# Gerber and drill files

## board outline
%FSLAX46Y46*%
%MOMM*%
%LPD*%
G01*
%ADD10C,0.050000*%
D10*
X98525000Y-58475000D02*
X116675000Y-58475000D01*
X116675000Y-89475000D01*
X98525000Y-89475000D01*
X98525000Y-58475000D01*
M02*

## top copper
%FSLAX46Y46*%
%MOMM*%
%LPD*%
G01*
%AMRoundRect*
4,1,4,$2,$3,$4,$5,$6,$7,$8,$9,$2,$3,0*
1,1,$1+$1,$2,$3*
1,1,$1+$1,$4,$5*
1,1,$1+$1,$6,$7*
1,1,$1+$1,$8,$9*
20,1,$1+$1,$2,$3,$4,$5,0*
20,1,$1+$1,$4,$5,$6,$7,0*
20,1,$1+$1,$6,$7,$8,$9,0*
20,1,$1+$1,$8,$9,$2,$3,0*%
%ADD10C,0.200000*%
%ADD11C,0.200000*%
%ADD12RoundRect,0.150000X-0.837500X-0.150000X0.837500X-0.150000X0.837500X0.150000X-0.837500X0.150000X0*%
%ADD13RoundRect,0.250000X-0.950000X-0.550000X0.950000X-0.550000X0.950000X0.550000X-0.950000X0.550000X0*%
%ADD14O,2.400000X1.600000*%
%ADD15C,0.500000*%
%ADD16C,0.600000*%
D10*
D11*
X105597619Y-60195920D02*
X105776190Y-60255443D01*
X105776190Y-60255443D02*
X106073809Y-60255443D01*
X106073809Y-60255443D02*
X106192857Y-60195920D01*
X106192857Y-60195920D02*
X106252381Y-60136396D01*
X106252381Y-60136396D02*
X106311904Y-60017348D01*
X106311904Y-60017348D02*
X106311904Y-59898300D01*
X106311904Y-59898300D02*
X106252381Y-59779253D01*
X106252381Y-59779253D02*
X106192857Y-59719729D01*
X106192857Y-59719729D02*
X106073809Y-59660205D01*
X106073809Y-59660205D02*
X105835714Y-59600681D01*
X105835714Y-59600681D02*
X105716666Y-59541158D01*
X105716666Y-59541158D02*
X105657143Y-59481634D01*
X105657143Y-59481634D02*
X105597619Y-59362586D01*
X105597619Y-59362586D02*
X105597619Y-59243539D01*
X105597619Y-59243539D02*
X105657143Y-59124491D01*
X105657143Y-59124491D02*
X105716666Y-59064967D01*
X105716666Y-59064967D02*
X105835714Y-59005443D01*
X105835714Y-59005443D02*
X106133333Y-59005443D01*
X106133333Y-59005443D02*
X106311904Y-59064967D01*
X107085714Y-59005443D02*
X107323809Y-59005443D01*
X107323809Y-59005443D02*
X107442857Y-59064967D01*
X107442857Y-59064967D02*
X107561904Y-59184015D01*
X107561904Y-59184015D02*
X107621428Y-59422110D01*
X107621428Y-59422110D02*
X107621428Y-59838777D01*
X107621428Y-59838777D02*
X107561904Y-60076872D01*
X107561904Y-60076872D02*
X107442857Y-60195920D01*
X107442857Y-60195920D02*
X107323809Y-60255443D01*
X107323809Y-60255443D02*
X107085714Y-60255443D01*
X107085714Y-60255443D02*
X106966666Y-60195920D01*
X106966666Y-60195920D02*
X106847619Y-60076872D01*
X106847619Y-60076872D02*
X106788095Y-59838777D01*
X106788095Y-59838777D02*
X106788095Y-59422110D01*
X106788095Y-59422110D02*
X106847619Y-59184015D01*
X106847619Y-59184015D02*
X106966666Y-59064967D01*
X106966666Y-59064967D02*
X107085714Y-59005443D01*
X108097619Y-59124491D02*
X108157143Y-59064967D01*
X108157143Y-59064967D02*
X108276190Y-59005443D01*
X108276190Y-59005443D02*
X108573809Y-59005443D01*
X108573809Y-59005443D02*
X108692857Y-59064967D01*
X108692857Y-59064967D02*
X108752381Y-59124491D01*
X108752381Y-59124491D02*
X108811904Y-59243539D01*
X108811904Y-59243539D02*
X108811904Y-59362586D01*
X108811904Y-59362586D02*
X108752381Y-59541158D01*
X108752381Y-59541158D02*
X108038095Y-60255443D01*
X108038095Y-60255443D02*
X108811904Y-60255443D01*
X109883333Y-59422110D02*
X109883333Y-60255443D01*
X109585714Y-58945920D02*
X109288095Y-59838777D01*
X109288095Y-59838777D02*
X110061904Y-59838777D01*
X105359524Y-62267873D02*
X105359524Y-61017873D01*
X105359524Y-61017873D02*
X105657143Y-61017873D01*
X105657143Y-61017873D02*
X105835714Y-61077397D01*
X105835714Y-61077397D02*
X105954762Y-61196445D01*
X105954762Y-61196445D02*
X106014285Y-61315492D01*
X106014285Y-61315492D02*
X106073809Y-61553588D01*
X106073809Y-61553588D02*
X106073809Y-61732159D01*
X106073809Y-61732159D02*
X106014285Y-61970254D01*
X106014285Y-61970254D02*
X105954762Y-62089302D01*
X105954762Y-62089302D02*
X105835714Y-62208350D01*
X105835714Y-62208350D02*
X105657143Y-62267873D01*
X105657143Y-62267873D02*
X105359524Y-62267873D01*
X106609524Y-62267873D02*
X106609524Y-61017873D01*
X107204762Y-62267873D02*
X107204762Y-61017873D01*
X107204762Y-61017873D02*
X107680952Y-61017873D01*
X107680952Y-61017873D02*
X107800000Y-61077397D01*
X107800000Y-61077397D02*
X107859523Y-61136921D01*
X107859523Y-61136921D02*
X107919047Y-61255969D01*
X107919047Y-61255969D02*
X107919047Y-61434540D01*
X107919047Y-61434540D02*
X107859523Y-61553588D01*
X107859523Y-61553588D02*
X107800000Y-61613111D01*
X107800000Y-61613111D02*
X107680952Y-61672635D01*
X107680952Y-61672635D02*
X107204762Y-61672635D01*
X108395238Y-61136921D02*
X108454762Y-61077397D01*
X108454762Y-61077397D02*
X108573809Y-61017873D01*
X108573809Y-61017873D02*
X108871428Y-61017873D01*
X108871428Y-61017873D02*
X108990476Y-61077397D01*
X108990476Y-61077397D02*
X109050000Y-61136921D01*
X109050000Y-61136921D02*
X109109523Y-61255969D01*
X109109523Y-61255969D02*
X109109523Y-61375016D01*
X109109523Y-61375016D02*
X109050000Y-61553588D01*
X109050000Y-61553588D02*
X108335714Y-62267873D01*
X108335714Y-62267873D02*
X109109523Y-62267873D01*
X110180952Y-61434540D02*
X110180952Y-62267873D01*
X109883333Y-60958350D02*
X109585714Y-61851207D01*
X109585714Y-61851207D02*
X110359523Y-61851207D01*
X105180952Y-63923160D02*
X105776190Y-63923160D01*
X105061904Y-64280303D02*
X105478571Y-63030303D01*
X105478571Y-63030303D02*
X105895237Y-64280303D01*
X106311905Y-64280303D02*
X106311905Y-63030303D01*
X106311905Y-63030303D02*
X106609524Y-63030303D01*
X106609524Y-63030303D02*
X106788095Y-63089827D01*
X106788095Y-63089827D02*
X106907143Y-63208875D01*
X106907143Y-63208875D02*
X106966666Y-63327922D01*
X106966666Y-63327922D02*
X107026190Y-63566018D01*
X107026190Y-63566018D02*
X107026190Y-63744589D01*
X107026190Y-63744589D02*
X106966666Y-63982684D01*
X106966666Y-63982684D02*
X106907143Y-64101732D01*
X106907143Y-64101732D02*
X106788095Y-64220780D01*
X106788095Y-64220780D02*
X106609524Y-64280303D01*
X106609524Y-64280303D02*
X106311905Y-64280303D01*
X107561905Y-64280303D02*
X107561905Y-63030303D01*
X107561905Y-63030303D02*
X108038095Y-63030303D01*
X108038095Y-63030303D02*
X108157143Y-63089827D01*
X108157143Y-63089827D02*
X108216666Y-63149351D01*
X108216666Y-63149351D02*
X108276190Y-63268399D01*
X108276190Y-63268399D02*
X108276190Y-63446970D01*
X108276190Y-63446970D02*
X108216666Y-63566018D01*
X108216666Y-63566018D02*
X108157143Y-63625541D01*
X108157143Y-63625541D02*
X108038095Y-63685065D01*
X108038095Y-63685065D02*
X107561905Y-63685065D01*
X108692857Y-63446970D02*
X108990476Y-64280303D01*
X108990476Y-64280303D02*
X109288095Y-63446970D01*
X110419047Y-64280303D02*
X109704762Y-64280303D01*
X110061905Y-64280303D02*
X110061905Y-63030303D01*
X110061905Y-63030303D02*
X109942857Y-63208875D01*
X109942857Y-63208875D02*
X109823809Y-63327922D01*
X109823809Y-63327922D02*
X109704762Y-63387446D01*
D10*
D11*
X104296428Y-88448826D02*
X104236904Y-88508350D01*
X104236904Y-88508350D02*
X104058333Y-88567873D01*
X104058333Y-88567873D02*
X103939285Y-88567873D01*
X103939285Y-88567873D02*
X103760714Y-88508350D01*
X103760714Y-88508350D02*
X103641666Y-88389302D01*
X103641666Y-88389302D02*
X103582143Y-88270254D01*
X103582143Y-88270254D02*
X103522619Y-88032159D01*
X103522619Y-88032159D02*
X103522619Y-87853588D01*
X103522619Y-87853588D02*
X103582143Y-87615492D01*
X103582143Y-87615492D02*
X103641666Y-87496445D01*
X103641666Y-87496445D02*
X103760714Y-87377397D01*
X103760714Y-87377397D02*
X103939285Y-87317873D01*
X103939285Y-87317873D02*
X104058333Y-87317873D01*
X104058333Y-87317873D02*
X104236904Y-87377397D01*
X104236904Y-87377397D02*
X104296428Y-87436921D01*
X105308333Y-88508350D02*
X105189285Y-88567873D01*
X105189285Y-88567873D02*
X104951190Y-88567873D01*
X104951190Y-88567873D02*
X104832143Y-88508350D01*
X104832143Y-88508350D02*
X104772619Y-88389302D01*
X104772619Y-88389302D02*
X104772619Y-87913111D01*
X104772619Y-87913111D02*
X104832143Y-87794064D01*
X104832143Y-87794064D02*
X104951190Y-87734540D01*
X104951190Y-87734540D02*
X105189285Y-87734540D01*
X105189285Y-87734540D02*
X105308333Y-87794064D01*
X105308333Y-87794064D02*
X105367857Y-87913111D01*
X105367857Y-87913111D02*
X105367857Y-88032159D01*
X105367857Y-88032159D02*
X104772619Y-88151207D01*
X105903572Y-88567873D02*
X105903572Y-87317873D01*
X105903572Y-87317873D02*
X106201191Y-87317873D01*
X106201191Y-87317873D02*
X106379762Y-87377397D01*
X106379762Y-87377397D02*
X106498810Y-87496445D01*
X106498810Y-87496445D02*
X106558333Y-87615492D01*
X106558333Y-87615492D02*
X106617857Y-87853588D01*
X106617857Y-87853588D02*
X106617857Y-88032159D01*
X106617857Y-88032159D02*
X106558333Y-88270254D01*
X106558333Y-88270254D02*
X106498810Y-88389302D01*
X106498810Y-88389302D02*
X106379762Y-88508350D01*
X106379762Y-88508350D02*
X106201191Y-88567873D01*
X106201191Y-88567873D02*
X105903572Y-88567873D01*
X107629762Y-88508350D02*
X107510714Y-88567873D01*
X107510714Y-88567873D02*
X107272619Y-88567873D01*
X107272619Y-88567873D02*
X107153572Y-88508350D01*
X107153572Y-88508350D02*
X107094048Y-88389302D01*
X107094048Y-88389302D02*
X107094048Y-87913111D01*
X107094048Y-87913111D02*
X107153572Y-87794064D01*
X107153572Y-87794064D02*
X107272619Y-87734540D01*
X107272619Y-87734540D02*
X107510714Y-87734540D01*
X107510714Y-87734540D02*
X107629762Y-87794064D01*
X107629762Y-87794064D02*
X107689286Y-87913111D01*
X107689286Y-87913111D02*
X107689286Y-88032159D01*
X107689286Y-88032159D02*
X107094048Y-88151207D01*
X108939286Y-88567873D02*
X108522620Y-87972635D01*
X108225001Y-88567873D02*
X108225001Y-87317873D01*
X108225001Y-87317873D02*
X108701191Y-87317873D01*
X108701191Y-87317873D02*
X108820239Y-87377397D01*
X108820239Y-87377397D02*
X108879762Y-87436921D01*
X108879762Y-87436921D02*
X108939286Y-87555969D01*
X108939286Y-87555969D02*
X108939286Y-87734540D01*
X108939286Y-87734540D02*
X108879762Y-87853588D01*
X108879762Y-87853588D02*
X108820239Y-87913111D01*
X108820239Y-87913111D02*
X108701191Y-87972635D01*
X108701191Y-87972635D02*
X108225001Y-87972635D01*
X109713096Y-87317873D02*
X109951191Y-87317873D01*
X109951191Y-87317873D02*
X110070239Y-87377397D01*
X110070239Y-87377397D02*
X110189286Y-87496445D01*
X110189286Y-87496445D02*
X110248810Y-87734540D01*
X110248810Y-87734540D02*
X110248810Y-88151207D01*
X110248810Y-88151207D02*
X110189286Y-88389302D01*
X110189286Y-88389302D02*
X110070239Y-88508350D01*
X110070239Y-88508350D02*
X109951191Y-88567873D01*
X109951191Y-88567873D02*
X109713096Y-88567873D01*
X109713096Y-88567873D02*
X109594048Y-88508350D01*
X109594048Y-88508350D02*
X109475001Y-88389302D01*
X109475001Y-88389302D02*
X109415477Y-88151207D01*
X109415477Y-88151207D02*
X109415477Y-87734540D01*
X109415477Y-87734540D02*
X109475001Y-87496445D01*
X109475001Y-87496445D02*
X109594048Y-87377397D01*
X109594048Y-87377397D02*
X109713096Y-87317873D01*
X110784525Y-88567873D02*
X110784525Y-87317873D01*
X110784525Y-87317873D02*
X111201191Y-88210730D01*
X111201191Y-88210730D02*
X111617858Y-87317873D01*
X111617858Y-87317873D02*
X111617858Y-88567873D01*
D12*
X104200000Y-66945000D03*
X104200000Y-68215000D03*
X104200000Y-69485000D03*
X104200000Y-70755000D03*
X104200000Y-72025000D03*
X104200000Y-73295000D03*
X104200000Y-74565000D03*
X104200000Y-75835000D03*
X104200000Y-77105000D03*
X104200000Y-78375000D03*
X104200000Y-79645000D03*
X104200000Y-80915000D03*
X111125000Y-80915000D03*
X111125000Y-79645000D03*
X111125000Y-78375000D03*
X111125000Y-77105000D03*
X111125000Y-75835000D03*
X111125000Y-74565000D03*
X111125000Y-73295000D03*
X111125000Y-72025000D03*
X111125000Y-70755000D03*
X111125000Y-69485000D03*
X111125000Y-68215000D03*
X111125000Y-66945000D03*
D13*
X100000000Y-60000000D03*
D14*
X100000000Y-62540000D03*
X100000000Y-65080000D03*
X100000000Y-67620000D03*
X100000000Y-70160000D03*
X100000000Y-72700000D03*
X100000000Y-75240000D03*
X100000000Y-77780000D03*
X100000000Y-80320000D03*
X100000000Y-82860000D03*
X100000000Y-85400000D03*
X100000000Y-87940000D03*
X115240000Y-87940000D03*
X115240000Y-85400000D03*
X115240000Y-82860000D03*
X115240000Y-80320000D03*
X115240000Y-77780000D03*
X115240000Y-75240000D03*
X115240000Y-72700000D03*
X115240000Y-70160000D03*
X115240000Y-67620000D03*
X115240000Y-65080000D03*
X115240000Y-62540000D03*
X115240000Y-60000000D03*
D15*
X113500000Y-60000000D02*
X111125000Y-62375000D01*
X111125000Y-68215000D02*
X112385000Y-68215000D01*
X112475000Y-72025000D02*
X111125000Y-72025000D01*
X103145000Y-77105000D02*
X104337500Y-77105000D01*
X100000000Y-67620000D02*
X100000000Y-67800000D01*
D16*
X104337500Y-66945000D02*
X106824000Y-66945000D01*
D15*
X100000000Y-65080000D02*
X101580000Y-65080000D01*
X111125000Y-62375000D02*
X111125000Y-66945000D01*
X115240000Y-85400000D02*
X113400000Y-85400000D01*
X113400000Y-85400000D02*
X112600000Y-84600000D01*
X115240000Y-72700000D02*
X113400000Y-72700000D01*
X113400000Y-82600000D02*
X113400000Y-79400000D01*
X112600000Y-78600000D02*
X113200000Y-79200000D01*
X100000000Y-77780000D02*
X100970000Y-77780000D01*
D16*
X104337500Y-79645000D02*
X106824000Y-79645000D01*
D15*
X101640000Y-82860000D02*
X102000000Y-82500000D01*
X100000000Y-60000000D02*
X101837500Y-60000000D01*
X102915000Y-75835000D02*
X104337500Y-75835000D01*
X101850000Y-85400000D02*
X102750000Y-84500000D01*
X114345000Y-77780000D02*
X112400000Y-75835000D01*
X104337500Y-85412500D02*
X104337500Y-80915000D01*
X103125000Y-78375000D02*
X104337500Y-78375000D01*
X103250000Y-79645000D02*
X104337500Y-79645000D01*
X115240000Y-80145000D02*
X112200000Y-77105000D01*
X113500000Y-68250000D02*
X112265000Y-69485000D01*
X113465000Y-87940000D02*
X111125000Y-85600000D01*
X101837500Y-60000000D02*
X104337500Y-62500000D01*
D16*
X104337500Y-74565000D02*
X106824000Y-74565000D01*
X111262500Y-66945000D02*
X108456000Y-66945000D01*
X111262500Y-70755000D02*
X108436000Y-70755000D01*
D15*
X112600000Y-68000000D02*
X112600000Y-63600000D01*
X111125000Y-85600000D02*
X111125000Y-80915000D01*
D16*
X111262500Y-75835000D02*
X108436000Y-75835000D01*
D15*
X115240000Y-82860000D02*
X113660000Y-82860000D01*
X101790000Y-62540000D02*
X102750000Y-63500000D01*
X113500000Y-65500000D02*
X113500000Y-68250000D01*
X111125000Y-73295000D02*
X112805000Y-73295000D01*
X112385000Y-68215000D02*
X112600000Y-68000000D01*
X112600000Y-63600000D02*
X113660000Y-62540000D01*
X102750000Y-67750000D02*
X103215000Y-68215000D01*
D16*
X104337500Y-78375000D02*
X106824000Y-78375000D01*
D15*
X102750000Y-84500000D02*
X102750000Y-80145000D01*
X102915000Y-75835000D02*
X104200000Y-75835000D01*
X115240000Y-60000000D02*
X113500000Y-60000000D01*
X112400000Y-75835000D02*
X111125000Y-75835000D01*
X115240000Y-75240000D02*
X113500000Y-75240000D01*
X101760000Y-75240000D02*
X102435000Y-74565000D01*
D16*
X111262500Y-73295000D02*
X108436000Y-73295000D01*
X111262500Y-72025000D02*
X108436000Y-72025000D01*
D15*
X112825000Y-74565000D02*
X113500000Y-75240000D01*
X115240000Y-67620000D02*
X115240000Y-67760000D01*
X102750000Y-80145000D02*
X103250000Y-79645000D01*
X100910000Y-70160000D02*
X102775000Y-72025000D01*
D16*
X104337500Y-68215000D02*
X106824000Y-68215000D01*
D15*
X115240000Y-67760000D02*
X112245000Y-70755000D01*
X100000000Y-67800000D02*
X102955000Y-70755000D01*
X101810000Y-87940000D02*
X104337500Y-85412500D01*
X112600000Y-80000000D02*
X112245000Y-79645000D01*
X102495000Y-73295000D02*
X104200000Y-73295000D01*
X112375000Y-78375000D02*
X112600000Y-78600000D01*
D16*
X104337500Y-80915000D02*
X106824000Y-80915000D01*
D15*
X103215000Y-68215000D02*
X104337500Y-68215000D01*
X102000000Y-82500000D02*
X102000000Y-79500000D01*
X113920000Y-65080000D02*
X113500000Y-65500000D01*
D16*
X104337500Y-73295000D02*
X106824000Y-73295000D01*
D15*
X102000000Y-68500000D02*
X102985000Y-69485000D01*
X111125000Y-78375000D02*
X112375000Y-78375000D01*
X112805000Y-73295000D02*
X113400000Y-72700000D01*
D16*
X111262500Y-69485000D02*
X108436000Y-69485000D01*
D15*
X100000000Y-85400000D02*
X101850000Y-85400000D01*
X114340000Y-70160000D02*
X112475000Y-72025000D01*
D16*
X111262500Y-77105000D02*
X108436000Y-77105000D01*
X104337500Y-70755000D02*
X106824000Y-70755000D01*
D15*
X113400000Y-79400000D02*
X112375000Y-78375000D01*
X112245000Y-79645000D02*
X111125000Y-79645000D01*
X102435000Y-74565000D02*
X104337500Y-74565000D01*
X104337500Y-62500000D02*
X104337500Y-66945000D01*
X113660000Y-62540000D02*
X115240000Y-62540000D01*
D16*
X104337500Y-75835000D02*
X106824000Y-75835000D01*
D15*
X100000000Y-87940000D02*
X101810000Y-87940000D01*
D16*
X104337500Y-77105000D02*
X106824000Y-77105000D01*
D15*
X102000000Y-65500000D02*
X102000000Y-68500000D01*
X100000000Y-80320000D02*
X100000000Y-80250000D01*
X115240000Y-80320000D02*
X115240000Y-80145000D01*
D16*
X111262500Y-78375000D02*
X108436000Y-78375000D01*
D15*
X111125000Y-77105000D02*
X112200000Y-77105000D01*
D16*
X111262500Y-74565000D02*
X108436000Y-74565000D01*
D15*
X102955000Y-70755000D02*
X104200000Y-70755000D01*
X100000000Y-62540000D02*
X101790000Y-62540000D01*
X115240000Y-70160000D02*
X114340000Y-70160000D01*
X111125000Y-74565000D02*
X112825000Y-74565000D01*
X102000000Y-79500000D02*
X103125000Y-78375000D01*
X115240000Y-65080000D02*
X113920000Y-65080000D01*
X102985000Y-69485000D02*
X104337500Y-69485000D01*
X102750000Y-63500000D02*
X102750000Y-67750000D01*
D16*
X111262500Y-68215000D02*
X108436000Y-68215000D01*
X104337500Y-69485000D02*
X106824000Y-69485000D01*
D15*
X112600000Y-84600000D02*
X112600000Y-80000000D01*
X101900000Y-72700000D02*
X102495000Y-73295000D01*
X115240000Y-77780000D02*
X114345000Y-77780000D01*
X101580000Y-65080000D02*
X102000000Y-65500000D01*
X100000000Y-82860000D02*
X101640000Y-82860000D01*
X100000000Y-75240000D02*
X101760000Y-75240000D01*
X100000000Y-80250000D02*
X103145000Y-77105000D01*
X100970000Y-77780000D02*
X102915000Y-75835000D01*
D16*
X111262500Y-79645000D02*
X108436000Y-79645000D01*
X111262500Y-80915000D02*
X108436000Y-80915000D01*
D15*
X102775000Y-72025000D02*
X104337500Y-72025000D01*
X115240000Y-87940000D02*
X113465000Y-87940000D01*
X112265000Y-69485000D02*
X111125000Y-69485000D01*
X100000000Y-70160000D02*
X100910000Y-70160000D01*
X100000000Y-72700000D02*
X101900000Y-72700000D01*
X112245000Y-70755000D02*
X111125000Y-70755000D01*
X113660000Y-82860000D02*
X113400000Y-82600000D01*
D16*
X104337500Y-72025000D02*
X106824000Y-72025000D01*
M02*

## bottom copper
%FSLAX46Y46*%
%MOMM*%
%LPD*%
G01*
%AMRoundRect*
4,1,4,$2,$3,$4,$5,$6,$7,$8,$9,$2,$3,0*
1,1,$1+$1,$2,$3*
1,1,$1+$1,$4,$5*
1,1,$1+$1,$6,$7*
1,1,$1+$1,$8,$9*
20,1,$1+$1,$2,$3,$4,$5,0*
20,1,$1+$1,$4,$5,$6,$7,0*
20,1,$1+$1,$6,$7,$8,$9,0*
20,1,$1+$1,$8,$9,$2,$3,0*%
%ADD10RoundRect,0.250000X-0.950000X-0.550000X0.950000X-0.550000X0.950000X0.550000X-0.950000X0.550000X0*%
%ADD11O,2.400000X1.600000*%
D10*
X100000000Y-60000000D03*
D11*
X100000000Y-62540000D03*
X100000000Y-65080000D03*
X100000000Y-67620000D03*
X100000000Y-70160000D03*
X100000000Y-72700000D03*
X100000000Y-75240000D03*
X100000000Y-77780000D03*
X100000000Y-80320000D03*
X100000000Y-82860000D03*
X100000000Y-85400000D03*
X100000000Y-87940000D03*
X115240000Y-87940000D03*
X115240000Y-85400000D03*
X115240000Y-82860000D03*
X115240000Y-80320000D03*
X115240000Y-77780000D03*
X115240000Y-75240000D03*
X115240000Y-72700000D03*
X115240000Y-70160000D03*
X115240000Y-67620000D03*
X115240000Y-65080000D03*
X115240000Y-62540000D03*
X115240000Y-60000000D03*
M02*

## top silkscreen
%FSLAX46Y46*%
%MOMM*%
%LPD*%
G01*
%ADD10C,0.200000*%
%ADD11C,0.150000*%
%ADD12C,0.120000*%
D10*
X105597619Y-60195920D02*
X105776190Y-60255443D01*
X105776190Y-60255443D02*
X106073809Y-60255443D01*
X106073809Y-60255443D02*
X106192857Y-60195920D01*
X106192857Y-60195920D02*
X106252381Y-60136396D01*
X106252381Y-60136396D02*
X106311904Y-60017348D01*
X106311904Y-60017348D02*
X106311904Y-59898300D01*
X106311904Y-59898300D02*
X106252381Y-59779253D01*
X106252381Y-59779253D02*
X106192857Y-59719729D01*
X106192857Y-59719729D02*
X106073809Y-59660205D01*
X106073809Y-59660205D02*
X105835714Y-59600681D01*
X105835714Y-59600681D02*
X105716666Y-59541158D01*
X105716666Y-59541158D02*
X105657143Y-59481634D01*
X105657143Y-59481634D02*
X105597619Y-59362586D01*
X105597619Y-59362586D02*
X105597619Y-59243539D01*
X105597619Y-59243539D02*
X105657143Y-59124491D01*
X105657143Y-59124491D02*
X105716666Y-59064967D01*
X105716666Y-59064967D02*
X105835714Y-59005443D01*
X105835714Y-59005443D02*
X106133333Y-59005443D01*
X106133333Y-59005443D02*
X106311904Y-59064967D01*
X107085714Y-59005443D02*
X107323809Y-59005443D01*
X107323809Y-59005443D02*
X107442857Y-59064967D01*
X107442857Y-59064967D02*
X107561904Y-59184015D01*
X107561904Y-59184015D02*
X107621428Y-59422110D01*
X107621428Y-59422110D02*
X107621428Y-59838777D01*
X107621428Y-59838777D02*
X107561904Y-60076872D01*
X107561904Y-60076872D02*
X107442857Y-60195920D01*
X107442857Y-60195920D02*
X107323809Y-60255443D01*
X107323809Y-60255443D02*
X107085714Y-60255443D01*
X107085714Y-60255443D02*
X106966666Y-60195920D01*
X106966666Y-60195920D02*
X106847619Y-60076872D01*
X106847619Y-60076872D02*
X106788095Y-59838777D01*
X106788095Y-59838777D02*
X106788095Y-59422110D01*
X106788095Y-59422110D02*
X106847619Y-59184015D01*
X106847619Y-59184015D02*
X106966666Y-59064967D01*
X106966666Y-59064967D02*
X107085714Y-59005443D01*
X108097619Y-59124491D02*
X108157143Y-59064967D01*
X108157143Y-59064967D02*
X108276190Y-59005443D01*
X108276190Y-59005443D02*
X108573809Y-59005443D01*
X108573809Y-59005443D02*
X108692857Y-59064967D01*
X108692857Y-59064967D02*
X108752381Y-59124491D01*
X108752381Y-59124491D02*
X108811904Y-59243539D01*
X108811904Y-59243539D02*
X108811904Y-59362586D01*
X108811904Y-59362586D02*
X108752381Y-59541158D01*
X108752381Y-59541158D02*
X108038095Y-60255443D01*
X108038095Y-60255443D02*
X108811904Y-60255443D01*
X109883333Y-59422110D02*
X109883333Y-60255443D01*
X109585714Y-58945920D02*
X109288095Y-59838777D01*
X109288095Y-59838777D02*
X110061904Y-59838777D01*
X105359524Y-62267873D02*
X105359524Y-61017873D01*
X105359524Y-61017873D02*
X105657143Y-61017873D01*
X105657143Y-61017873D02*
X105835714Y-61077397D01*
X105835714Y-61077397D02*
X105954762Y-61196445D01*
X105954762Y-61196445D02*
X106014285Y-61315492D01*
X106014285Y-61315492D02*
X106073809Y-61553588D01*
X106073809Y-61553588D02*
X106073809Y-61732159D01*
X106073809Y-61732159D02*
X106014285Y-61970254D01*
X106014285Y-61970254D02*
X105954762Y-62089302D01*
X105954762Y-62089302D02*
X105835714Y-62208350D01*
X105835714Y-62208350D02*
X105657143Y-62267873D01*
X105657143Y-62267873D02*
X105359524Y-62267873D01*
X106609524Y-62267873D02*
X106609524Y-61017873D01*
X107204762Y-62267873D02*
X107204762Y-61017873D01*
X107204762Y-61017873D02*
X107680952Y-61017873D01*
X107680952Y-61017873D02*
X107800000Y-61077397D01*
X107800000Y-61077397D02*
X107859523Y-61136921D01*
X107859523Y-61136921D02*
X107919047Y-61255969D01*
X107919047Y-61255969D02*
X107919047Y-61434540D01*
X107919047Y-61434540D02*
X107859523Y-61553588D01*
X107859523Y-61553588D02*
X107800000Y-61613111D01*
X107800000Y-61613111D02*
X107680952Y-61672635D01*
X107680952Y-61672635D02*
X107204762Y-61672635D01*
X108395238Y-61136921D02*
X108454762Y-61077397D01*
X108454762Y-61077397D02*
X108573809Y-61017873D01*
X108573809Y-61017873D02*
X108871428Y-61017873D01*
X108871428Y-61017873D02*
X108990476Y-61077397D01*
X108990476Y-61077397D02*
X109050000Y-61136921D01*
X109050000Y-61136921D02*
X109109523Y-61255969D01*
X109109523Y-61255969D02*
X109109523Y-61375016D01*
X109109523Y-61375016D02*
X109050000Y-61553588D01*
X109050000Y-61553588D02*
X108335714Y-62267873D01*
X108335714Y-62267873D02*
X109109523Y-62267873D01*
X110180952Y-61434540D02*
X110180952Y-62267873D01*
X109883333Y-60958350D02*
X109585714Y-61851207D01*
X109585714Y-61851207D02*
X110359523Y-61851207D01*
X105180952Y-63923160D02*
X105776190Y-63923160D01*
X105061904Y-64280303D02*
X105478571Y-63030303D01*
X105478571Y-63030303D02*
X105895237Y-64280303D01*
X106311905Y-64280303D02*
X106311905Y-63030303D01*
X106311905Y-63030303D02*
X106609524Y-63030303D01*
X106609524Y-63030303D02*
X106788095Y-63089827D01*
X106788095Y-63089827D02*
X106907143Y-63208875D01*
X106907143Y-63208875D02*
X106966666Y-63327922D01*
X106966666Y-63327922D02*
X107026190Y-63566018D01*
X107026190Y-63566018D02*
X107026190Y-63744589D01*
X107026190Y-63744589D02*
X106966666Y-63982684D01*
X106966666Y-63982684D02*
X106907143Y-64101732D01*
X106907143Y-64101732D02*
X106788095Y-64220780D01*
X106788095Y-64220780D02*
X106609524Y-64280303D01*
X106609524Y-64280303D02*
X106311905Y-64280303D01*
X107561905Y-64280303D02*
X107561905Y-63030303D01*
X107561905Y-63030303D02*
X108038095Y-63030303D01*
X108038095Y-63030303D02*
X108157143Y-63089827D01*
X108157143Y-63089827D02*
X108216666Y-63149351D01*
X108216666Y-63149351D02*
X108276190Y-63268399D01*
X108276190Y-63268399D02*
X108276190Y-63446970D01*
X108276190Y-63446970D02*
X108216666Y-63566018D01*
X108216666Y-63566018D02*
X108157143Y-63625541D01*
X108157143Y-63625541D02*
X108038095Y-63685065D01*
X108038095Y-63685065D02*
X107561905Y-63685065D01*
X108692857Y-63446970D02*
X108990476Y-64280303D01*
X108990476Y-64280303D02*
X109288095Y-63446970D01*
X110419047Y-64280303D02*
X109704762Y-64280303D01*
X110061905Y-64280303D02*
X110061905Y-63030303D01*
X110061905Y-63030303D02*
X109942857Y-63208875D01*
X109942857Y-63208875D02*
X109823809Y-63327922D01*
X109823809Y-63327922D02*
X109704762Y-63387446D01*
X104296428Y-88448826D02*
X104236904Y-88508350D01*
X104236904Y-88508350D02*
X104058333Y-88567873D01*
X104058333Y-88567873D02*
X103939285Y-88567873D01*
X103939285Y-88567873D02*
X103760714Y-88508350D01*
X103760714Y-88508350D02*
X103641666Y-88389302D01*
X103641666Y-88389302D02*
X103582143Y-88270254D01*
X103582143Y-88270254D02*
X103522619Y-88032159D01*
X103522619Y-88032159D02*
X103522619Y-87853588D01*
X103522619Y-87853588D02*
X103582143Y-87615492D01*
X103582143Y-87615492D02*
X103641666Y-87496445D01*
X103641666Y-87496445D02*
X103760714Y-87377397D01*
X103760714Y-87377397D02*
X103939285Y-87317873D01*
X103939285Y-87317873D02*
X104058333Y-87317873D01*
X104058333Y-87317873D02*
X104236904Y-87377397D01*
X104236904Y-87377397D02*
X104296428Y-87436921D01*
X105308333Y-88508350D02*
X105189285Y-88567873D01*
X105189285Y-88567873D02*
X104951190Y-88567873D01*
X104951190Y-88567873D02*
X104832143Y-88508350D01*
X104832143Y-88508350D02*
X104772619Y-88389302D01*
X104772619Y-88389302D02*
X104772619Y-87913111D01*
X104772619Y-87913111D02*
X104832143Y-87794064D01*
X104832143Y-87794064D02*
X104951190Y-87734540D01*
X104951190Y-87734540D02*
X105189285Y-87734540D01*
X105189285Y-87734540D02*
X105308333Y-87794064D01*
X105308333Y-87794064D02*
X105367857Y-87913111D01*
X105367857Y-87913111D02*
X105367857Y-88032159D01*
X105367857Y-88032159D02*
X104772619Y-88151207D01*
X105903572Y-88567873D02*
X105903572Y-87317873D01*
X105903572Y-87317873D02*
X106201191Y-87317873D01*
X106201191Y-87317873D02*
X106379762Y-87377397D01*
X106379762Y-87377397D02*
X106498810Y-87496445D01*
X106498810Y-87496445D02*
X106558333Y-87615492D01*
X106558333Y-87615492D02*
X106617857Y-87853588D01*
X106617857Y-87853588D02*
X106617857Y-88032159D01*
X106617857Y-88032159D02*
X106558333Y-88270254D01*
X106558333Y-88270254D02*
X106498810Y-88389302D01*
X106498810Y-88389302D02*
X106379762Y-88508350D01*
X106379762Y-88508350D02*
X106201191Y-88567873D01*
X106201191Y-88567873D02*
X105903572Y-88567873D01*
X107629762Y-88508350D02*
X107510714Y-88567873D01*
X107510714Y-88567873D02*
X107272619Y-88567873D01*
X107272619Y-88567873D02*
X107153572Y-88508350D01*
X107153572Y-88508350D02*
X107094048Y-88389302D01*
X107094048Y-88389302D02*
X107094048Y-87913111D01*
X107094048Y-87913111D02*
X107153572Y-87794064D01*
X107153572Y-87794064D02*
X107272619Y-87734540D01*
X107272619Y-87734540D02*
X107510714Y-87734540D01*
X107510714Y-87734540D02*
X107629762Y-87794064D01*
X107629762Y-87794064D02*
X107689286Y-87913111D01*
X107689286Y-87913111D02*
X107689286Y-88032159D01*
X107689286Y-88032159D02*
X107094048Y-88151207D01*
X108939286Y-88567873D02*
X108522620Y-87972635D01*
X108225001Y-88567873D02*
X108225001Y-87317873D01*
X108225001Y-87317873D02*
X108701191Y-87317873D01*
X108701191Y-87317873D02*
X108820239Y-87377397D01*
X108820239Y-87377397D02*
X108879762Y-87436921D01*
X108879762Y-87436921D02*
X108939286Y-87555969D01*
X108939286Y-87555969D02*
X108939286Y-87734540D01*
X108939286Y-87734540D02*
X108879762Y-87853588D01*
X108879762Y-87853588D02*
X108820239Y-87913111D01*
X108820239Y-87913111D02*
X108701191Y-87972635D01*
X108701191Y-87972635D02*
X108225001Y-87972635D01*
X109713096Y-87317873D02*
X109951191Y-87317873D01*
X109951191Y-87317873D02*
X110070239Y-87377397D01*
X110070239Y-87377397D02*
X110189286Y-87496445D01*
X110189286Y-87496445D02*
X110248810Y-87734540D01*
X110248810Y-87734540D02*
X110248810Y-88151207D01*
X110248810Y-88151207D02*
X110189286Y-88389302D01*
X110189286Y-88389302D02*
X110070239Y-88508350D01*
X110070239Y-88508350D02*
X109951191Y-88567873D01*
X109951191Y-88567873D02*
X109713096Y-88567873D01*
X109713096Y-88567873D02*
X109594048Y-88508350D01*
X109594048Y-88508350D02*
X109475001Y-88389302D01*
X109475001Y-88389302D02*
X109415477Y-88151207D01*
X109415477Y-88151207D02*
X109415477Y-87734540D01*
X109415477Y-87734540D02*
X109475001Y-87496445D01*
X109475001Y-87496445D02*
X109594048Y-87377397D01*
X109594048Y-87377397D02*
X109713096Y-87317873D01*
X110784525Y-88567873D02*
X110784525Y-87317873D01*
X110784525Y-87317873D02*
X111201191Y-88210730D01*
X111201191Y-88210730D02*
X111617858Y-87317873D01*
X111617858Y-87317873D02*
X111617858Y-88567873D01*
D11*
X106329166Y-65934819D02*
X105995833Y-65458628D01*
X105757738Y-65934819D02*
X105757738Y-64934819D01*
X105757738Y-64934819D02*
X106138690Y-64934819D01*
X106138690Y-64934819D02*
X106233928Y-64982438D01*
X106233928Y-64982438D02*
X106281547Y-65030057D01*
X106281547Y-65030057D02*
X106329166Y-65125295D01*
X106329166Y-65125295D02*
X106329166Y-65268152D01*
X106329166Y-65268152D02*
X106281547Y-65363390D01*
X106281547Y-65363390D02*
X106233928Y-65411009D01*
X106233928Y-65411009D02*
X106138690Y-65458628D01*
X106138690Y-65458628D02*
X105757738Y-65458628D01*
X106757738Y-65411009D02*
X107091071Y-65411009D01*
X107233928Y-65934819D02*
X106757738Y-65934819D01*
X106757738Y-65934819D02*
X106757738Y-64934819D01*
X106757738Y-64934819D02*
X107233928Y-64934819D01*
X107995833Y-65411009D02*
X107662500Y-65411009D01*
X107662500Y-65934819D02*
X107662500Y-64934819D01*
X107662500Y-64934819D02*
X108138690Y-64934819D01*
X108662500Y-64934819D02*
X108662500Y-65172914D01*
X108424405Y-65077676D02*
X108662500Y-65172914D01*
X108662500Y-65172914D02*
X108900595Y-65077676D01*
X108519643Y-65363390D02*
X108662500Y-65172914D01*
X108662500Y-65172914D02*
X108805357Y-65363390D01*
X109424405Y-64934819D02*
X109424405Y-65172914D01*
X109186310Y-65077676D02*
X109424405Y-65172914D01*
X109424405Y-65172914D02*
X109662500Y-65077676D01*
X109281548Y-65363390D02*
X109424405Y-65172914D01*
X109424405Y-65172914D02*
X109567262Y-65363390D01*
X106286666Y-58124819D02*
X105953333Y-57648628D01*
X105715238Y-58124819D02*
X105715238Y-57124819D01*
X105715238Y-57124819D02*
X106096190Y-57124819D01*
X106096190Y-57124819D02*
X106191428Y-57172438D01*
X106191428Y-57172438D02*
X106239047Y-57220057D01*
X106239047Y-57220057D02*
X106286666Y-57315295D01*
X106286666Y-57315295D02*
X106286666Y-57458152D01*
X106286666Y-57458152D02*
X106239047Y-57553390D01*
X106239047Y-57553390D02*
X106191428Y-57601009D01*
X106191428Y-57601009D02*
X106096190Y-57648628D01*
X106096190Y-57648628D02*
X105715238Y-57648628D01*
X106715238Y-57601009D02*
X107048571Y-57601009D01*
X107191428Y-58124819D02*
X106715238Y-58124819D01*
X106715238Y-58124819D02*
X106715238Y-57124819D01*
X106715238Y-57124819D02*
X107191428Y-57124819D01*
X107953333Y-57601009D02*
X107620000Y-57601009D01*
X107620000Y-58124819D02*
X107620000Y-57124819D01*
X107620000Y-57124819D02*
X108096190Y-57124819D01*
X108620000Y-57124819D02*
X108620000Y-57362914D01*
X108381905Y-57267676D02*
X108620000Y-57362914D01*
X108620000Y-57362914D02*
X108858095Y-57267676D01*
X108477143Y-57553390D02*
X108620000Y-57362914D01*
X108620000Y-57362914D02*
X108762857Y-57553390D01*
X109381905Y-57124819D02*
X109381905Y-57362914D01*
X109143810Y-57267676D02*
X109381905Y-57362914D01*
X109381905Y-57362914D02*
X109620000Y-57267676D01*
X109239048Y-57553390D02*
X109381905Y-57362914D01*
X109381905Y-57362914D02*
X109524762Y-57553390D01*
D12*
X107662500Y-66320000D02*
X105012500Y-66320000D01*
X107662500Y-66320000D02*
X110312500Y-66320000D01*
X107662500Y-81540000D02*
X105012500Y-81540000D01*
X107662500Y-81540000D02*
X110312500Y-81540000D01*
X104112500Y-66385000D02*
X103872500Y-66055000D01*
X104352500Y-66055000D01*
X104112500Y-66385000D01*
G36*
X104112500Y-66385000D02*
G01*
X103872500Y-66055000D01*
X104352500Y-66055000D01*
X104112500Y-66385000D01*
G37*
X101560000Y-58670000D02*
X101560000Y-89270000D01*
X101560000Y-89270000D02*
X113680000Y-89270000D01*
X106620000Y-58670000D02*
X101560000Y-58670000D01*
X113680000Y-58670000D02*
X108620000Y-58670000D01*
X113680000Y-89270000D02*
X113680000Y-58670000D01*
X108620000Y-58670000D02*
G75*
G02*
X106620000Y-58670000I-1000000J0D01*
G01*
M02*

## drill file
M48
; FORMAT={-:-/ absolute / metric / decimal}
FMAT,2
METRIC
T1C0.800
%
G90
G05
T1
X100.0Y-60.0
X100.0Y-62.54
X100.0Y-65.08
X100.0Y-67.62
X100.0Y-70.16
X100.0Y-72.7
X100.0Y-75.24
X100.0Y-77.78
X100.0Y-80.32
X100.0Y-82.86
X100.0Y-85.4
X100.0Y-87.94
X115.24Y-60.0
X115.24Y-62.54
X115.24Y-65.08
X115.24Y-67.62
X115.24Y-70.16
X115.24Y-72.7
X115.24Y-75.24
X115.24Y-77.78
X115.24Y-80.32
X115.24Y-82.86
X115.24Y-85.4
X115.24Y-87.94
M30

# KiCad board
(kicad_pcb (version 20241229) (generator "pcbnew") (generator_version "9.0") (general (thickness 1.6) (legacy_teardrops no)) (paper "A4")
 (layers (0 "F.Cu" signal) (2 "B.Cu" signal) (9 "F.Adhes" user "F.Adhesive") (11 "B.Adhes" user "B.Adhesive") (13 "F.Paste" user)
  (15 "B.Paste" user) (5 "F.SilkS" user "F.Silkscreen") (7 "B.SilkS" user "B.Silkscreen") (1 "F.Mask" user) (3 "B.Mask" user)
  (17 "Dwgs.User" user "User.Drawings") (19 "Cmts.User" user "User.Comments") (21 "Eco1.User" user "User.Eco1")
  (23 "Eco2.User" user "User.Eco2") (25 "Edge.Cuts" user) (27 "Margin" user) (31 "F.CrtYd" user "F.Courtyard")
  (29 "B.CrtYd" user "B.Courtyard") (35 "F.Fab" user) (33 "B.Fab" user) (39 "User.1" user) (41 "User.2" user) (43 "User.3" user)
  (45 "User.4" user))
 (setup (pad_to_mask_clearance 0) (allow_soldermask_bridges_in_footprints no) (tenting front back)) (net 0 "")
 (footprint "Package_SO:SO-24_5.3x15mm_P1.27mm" (layer "F.Cu") (at 107.6625 73.93)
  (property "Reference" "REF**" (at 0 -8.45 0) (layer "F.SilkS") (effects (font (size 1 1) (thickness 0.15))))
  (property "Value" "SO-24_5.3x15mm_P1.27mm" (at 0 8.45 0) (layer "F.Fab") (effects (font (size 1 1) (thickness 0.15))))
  (fp_line (start 0 -7.61) (end -2.65 -7.61) (stroke (width 0.12) (type solid)) (layer "F.SilkS"))
  (fp_line (start 0 -7.61) (end 2.65 -7.61) (stroke (width 0.12) (type solid)) (layer "F.SilkS"))
  (fp_line (start 0 7.61) (end -2.65 7.61) (stroke (width 0.12) (type solid)) (layer "F.SilkS"))
  (fp_line (start 0 7.61) (end 2.65 7.61) (stroke (width 0.12) (type solid)) (layer "F.SilkS"))
  (fp_poly (pts (xy -3.55 -7.545) (xy -3.79 -7.875) (xy -3.31 -7.875)) (stroke (width 0.12) (type solid)) (fill yes) (layer "F.SilkS"))
  (pad "1" smd roundrect (at -3.4625 -6.985) (size 1.975 0.6) (layers "F.Cu" "F.Mask" "F.Paste") (roundrect_rratio 0.25))
  (pad "2" smd roundrect (at -3.4625 -5.715) (size 1.975 0.6) (layers "F.Cu" "F.Mask" "F.Paste") (roundrect_rratio 0.25))
  (pad "3" smd roundrect (at -3.4625 -4.445) (size 1.975 0.6) (layers "F.Cu" "F.Mask" "F.Paste") (roundrect_rratio 0.25))
  (pad "4" smd roundrect (at -3.4625 -3.175) (size 1.975 0.6) (layers "F.Cu" "F.Mask" "F.Paste") (roundrect_rratio 0.25))
  (pad "5" smd roundrect (at -3.4625 -1.905) (size 1.975 0.6) (layers "F.Cu" "F.Mask" "F.Paste") (roundrect_rratio 0.25))
  (pad "6" smd roundrect (at -3.4625 -0.635) (size 1.975 0.6) (layers "F.Cu" "F.Mask" "F.Paste") (roundrect_rratio 0.25))
  (pad "7" smd roundrect (at -3.4625 0.635) (size 1.975 0.6) (layers "F.Cu" "F.Mask" "F.Paste") (roundrect_rratio 0.25))
  (pad "8" smd roundrect (at -3.4625 1.905) (size 1.975 0.6) (layers "F.Cu" "F.Mask" "F.Paste") (roundrect_rratio 0.25))
  (pad "9" smd roundrect (at -3.4625 3.175) (size 1.975 0.6) (layers "F.Cu" "F.Mask" "F.Paste") (roundrect_rratio 0.25))
  (pad "10" smd roundrect (at -3.4625 4.445) (size 1.975 0.6) (layers "F.Cu" "F.Mask" "F.Paste") (roundrect_rratio 0.25))
  (pad "11" smd roundrect (at -3.4625 5.715) (size 1.975 0.6) (layers "F.Cu" "F.Mask" "F.Paste") (roundrect_rratio 0.25))
  (pad "12" smd roundrect (at -3.4625 6.985) (size 1.975 0.6) (layers "F.Cu" "F.Mask" "F.Paste") (roundrect_rratio 0.25))
  (pad "13" smd roundrect (at 3.4625 6.985) (size 1.975 0.6) (layers "F.Cu" "F.Mask" "F.Paste") (roundrect_rratio 0.25))
  (pad "14" smd roundrect (at 3.4625 5.715) (size 1.975 0.6) (layers "F.Cu" "F.Mask" "F.Paste") (roundrect_rratio 0.25))
  (pad "15" smd roundrect (at 3.4625 4.445) (size 1.975 0.6) (layers "F.Cu" "F.Mask" "F.Paste") (roundrect_rratio 0.25))
  (pad "16" smd roundrect (at 3.4625 3.175) (size 1.975 0.6) (layers "F.Cu" "F.Mask" "F.Paste") (roundrect_rratio 0.25))
  (pad "17" smd roundrect (at 3.4625 1.905) (size 1.975 0.6) (layers "F.Cu" "F.Mask" "F.Paste") (roundrect_rratio 0.25))
  (pad "18" smd roundrect (at 3.4625 0.635) (size 1.975 0.6) (layers "F.Cu" "F.Mask" "F.Paste") (roundrect_rratio 0.25))
  (pad "19" smd roundrect (at 3.4625 -0.635) (size 1.975 0.6) (layers "F.Cu" "F.Mask" "F.Paste") (roundrect_rratio 0.25))
  (pad "20" smd roundrect (at 3.4625 -1.905) (size 1.975 0.6) (layers "F.Cu" "F.Mask" "F.Paste") (roundrect_rratio 0.25))
  (pad "21" smd roundrect (at 3.4625 -3.175) (size 1.975 0.6) (layers "F.Cu" "F.Mask" "F.Paste") (roundrect_rratio 0.25))
  (pad "22" smd roundrect (at 3.4625 -4.445) (size 1.975 0.6) (layers "F.Cu" "F.Mask" "F.Paste") (roundrect_rratio 0.25))
  (pad "23" smd roundrect (at 3.4625 -5.715) (size 1.975 0.6) (layers "F.Cu" "F.Mask" "F.Paste") (roundrect_rratio 0.25))
  (pad "24" smd roundrect (at 3.4625 -6.985) (size 1.975 0.6) (layers "F.Cu" "F.Mask" "F.Paste") (roundrect_rratio 0.25)))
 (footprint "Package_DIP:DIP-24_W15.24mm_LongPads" (layer "F.Cu") (at 100 60)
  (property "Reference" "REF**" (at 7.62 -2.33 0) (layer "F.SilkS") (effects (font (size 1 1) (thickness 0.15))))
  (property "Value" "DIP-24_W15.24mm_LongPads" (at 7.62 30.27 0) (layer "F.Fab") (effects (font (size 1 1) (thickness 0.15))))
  (fp_line (start 1.56 -1.33) (end 1.56 29.27) (stroke (width 0.12) (type solid)) (layer "F.SilkS"))
  (fp_line (start 1.56 29.27) (end 13.68 29.27) (stroke (width 0.12) (type solid)) (layer "F.SilkS"))
  (fp_line (start 6.62 -1.33) (end 1.56 -1.33) (stroke (width 0.12) (type solid)) (layer "F.SilkS"))
  (fp_line (start 13.68 -1.33) (end 8.62 -1.33) (stroke (width 0.12) (type solid)) (layer "F.SilkS"))
  (fp_line (start 13.68 29.27) (end 13.68 -1.33) (stroke (width 0.12) (type solid)) (layer "F.SilkS"))
  (fp_arc (start 8.62 -1.33) (mid 7.62 -0.33) (end 6.62 -1.33) (stroke (width 0.12) (type solid)) (layer "F.SilkS"))
  (pad "1" thru_hole roundrect (at 0 0) (size 2.4 1.6) (drill 0.8) (layers "*.Cu" "*.Mask") (remove_unused_layers no)
   (roundrect_rratio 0.15625))
  (pad "2" thru_hole oval (at 0 2.54) (size 2.4 1.6) (drill 0.8) (layers "*.Cu" "*.Mask") (remove_unused_layers no))
  (pad "3" thru_hole oval (at 0 5.08) (size 2.4 1.6) (drill 0.8) (layers "*.Cu" "*.Mask") (remove_unused_layers no))
  (pad "4" thru_hole oval (at 0 7.62) (size 2.4 1.6) (drill 0.8) (layers "*.Cu" "*.Mask") (remove_unused_layers no))
  (pad "5" thru_hole oval (at 0 10.16) (size 2.4 1.6) (drill 0.8) (layers "*.Cu" "*.Mask") (remove_unused_layers no))
  (pad "6" thru_hole oval (at 0 12.7) (size 2.4 1.6) (drill 0.8) (layers "*.Cu" "*.Mask") (remove_unused_layers no))
  (pad "7" thru_hole oval (at 0 15.24) (size 2.4 1.6) (drill 0.8) (layers "*.Cu" "*.Mask") (remove_unused_layers no))
  (pad "8" thru_hole oval (at 0 17.78) (size 2.4 1.6) (drill 0.8) (layers "*.Cu" "*.Mask") (remove_unused_layers no))
  (pad "9" thru_hole oval (at 0 20.32) (size 2.4 1.6) (drill 0.8) (layers "*.Cu" "*.Mask") (remove_unused_layers no))
  (pad "10" thru_hole oval (at 0 22.86) (size 2.4 1.6) (drill 0.8) (layers "*.Cu" "*.Mask") (remove_unused_layers no))
  (pad "11" thru_hole oval (at 0 25.4) (size 2.4 1.6) (drill 0.8) (layers "*.Cu" "*.Mask") (remove_unused_layers no))
  (pad "12" thru_hole oval (at 0 27.94) (size 2.4 1.6) (drill 0.8) (layers "*.Cu" "*.Mask") (remove_unused_layers no))
  (pad "13" thru_hole oval (at 15.24 27.94) (size 2.4 1.6) (drill 0.8) (layers "*.Cu" "*.Mask") (remove_unused_layers no))
  (pad "14" thru_hole oval (at 15.24 25.4) (size 2.4 1.6) (drill 0.8) (layers "*.Cu" "*.Mask") (remove_unused_layers no))
  (pad "15" thru_hole oval (at 15.24 22.86) (size 2.4 1.6) (drill 0.8) (layers "*.Cu" "*.Mask") (remove_unused_layers no))
  (pad "16" thru_hole oval (at 15.24 20.32) (size 2.4 1.6) (drill 0.8) (layers "*.Cu" "*.Mask") (remove_unused_layers no))
  (pad "17" thru_hole oval (at 15.24 17.78) (size 2.4 1.6) (drill 0.8) (layers "*.Cu" "*.Mask") (remove_unused_layers no))
  (pad "18" thru_hole oval (at 15.24 15.24) (size 2.4 1.6) (drill 0.8) (layers "*.Cu" "*.Mask") (remove_unused_layers no))
  (pad "19" thru_hole oval (at 15.24 12.7) (size 2.4 1.6) (drill 0.8) (layers "*.Cu" "*.Mask") (remove_unused_layers no))
  (pad "20" thru_hole oval (at 15.24 10.16) (size 2.4 1.6) (drill 0.8) (layers "*.Cu" "*.Mask") (remove_unused_layers no))
  (pad "21" thru_hole oval (at 15.24 7.62) (size 2.4 1.6) (drill 0.8) (layers "*.Cu" "*.Mask") (remove_unused_layers no))
  (pad "22" thru_hole oval (at 15.24 5.08) (size 2.4 1.6) (drill 0.8) (layers "*.Cu" "*.Mask") (remove_unused_layers no))
  (pad "23" thru_hole oval (at 15.24 2.54) (size 2.4 1.6) (drill 0.8) (layers "*.Cu" "*.Mask") (remove_unused_layers no))
  (pad "24" thru_hole oval (at 15.24 0) (size 2.4 1.6) (drill 0.8) (layers "*.Cu" "*.Mask") (remove_unused_layers no)))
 (gr_rect (start 98.525 58.475) (end 116.675 89.475) (stroke (width 0.05) (type default)) (fill no) (layer "Edge.Cuts"))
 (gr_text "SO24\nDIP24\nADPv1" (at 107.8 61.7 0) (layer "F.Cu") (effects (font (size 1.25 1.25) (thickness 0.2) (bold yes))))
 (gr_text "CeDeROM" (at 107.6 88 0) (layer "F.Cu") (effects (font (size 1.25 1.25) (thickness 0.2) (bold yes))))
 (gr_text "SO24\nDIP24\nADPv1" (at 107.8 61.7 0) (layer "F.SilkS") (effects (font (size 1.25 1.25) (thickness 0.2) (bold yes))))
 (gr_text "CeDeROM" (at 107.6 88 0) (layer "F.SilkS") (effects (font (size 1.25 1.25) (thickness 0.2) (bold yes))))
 (segment (start 113.5 60) (end 111.125 62.375) (width 0.5) (layer "F.Cu") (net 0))
 (segment (start 111.125 68.215) (end 112.385 68.215) (width 0.5) (layer "F.Cu") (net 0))
 (segment (start 112.475 72.025) (end 111.125 72.025) (width 0.5) (layer "F.Cu") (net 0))
 (segment (start 103.145 77.105) (end 104.3375 77.105) (width 0.5) (layer "F.Cu") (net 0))
 (segment (start 100 67.62) (end 100 67.8) (width 0.5) (layer "F.Cu") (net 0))
 (segment (start 104.3375 66.945) (end 106.824 66.945) (width 0.6) (layer "F.Cu") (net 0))
 (segment (start 100 65.08) (end 101.58 65.08) (width 0.5) (layer "F.Cu") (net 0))
 (segment (start 111.125 62.375) (end 111.125 66.945) (width 0.5) (layer "F.Cu") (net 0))
 (segment (start 115.24 85.4) (end 113.4 85.4) (width 0.5) (layer "F.Cu") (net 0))
 (segment (start 113.4 85.4) (end 112.6 84.6) (width 0.5) (layer "F.Cu") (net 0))
 (segment (start 115.24 72.7) (end 113.4 72.7) (width 0.5) (layer "F.Cu") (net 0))
 (segment (start 113.4 82.6) (end 113.4 79.4) (width 0.5) (layer "F.Cu") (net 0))
 (segment (start 112.6 78.6) (end 113.2 79.2) (width 0.5) (layer "F.Cu") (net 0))
 (segment (start 100 77.78) (end 100.97 77.78) (width 0.5) (layer "F.Cu") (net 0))
 (segment (start 104.3375 79.645) (end 106.824 79.645) (width 0.6) (layer "F.Cu") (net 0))
 (segment (start 101.64 82.86) (end 102 82.5) (width 0.5) (layer "F.Cu") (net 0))
 (segment (start 100 60) (end 101.8375 60) (width 0.5) (layer "F.Cu") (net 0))
 (segment (start 102.915 75.835) (end 104.3375 75.835) (width 0.5) (layer "F.Cu") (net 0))
 (segment (start 101.85 85.4) (end 102.75 84.5) (width 0.5) (layer "F.Cu") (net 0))
 (segment (start 114.345 77.78) (end 112.4 75.835) (width 0.5) (layer "F.Cu") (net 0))
 (segment (start 104.3375 85.4125) (end 104.3375 80.915) (width 0.5) (layer "F.Cu") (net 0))
 (segment (start 103.125 78.375) (end 104.3375 78.375) (width 0.5) (layer "F.Cu") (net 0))
 (segment (start 103.25 79.645) (end 104.3375 79.645) (width 0.5) (layer "F.Cu") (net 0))
 (segment (start 115.24 80.145) (end 112.2 77.105) (width 0.5) (layer "F.Cu") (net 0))
 (segment (start 113.5 68.25) (end 112.265 69.485) (width 0.5) (layer "F.Cu") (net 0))
 (segment (start 113.465 87.94) (end 111.125 85.6) (width 0.5) (layer "F.Cu") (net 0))
 (segment (start 101.8375 60) (end 104.3375 62.5) (width 0.5) (layer "F.Cu") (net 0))
 (segment (start 104.3375 74.565) (end 106.824 74.565) (width 0.6) (layer "F.Cu") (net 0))
 (segment (start 111.2625 66.945) (end 108.456 66.945) (width 0.6) (layer "F.Cu") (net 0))
 (segment (start 111.2625 70.755) (end 108.436 70.755) (width 0.6) (layer "F.Cu") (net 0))
 (segment (start 112.6 68) (end 112.6 63.6) (width 0.5) (layer "F.Cu") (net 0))
 (segment (start 111.125 85.6) (end 111.125 80.915) (width 0.5) (layer "F.Cu") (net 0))
 (segment (start 111.2625 75.835) (end 108.436 75.835) (width 0.6) (layer "F.Cu") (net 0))
 (segment (start 115.24 82.86) (end 113.66 82.86) (width 0.5) (layer "F.Cu") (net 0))
 (segment (start 101.79 62.54) (end 102.75 63.5) (width 0.5) (layer "F.Cu") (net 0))
 (segment (start 113.5 65.5) (end 113.5 68.25) (width 0.5) (layer "F.Cu") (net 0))
 (segment (start 111.125 73.295) (end 112.805 73.295) (width 0.5) (layer "F.Cu") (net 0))
 (segment (start 112.385 68.215) (end 112.6 68) (width 0.5) (layer "F.Cu") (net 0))
 (segment (start 112.6 63.6) (end 113.66 62.54) (width 0.5) (layer "F.Cu") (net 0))
 (segment (start 102.75 67.75) (end 103.215 68.215) (width 0.5) (layer "F.Cu") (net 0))
 (segment (start 104.3375 78.375) (end 106.824 78.375) (width 0.6) (layer "F.Cu") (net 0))
 (segment (start 102.75 84.5) (end 102.75 80.145) (width 0.5) (layer "F.Cu") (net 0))
 (segment (start 102.915 75.835) (end 104.2 75.835) (width 0.5) (layer "F.Cu") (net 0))
 (segment (start 115.24 60) (end 113.5 60) (width 0.5) (layer "F.Cu") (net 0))
 (segment (start 112.4 75.835) (end 111.125 75.835) (width 0.5) (layer "F.Cu") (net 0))
 (segment (start 115.24 75.24) (end 113.5 75.24) (width 0.5) (layer "F.Cu") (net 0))
 (segment (start 101.76 75.24) (end 102.435 74.565) (width 0.5) (layer "F.Cu") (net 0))
 (segment (start 111.2625 73.295) (end 108.436 73.295) (width 0.6) (layer "F.Cu") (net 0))
 (segment (start 111.2625 72.025) (end 108.436 72.025) (width 0.6) (layer "F.Cu") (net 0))
 (segment (start 112.825 74.565) (end 113.5 75.24) (width 0.5) (layer "F.Cu") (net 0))
 (segment (start 115.24 67.62) (end 115.24 67.76) (width 0.5) (layer "F.Cu") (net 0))
 (segment (start 102.75 80.145) (end 103.25 79.645) (width 0.5) (layer "F.Cu") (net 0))
 (segment (start 100.91 70.16) (end 102.775 72.025) (width 0.5) (layer "F.Cu") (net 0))
 (segment (start 104.3375 68.215) (end 106.824 68.215) (width 0.6) (layer "F.Cu") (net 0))
 (segment (start 115.24 67.76) (end 112.245 70.755) (width 0.5) (layer "F.Cu") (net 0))
 (segment (start 100 67.8) (end 102.955 70.755) (width 0.5) (layer "F.Cu") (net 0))
 (segment (start 101.81 87.94) (end 104.3375 85.4125) (width 0.5) (layer "F.Cu") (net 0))
 (segment (start 112.6 80) (end 112.245 79.645) (width 0.5) (layer "F.Cu") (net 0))
 (segment (start 102.495 73.295) (end 104.2 73.295) (width 0.5) (layer "F.Cu") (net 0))
 (segment (start 112.375 78.375) (end 112.6 78.6) (width 0.5) (layer "F.Cu") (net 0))
 (segment (start 104.3375 80.915) (end 106.824 80.915) (width 0.6) (layer "F.Cu") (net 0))
 (segment (start 103.215 68.215) (end 104.3375 68.215) (width 0.5) (layer "F.Cu") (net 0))
 (segment (start 102 82.5) (end 102 79.5) (width 0.5) (layer "F.Cu") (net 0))
 (segment (start 113.92 65.08) (end 113.5 65.5) (width 0.5) (layer "F.Cu") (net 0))
 (segment (start 104.3375 73.295) (end 106.824 73.295) (width 0.6) (layer "F.Cu") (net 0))
 (segment (start 102 68.5) (end 102.985 69.485) (width 0.5) (layer "F.Cu") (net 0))
 (segment (start 111.125 78.375) (end 112.375 78.375) (width 0.5) (layer "F.Cu") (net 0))
 (segment (start 112.805 73.295) (end 113.4 72.7) (width 0.5) (layer "F.Cu") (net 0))
 (segment (start 111.2625 69.485) (end 108.436 69.485) (width 0.6) (layer "F.Cu") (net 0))
 (segment (start 100 85.4) (end 101.85 85.4) (width 0.5) (layer "F.Cu") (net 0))
 (segment (start 114.34 70.16) (end 112.475 72.025) (width 0.5) (layer "F.Cu") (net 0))
 (segment (start 111.2625 77.105) (end 108.436 77.105) (width 0.6) (layer "F.Cu") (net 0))
 (segment (start 104.3375 70.755) (end 106.824 70.755) (width 0.6) (layer "F.Cu") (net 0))
 (segment (start 113.4 79.4) (end 112.375 78.375) (width 0.5) (layer "F.Cu") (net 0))
 (segment (start 112.245 79.645) (end 111.125 79.645) (width 0.5) (layer "F.Cu") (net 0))
 (segment (start 102.435 74.565) (end 104.3375 74.565) (width 0.5) (layer "F.Cu") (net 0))
 (segment (start 104.3375 62.5) (end 104.3375 66.945) (width 0.5) (layer "F.Cu") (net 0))
 (segment (start 113.66 62.54) (end 115.24 62.54) (width 0.5) (layer "F.Cu") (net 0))
 (segment (start 104.3375 75.835) (end 106.824 75.835) (width 0.6) (layer "F.Cu") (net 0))
 (segment (start 100 87.94) (end 101.81 87.94) (width 0.5) (layer "F.Cu") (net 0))
 (segment (start 104.3375 77.105) (end 106.824 77.105) (width 0.6) (layer "F.Cu") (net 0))
 (segment (start 102 65.5) (end 102 68.5) (width 0.5) (layer "F.Cu") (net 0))
 (segment (start 100 80.32) (end 100 80.25) (width 0.5) (layer "F.Cu") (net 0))
 (segment (start 115.24 80.32) (end 115.24 80.145) (width 0.5) (layer "F.Cu") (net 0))
 (segment (start 111.2625 78.375) (end 108.436 78.375) (width 0.6) (layer "F.Cu") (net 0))
 (segment (start 111.125 77.105) (end 112.2 77.105) (width 0.5) (layer "F.Cu") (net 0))
 (segment (start 111.2625 74.565) (end 108.436 74.565) (width 0.6) (layer "F.Cu") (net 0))
 (segment (start 102.955 70.755) (end 104.2 70.755) (width 0.5) (layer "F.Cu") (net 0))
 (segment (start 100 62.54) (end 101.79 62.54) (width 0.5) (layer "F.Cu") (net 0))
 (segment (start 115.24 70.16) (end 114.34 70.16) (width 0.5) (layer "F.Cu") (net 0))
 (segment (start 111.125 74.565) (end 112.825 74.565) (width 0.5) (layer "F.Cu") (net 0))
 (segment (start 102 79.5) (end 103.125 78.375) (width 0.5) (layer "F.Cu") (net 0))
 (segment (start 115.24 65.08) (end 113.92 65.08) (width 0.5) (layer "F.Cu") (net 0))
 (segment (start 102.985 69.485) (end 104.3375 69.485) (width 0.5) (layer "F.Cu") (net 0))
 (segment (start 102.75 63.5) (end 102.75 67.75) (width 0.5) (layer "F.Cu") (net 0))
 (segment (start 111.2625 68.215) (end 108.436 68.215) (width 0.6) (layer "F.Cu") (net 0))
 (segment (start 104.3375 69.485) (end 106.824 69.485) (width 0.6) (layer "F.Cu") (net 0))
 (segment (start 112.6 84.6) (end 112.6 80) (width 0.5) (layer "F.Cu") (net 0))
 (segment (start 101.9 72.7) (end 102.495 73.295) (width 0.5) (layer "F.Cu") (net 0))
 (segment (start 115.24 77.78) (end 114.345 77.78) (width 0.5) (layer "F.Cu") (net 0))
 (segment (start 101.58 65.08) (end 102 65.5) (width 0.5) (layer "F.Cu") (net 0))
 (segment (start 100 82.86) (end 101.64 82.86) (width 0.5) (layer "F.Cu") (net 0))
 (segment (start 100 75.24) (end 101.76 75.24) (width 0.5) (layer "F.Cu") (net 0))
 (segment (start 100 80.25) (end 103.145 77.105) (width 0.5) (layer "F.Cu") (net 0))
 (segment (start 100.97 77.78) (end 102.915 75.835) (width 0.5) (layer "F.Cu") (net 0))
 (segment (start 111.2625 79.645) (end 108.436 79.645) (width 0.6) (layer "F.Cu") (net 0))
 (segment (start 111.2625 80.915) (end 108.436 80.915) (width 0.6) (layer "F.Cu") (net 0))
 (segment (start 102.775 72.025) (end 104.3375 72.025) (width 0.5) (layer "F.Cu") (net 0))
 (segment (start 115.24 87.94) (end 113.465 87.94) (width 0.5) (layer "F.Cu") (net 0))
 (segment (start 112.265 69.485) (end 111.125 69.485) (width 0.5) (layer "F.Cu") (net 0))
 (segment (start 100 70.16) (end 100.91 70.16) (width 0.5) (layer "F.Cu") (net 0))
 (segment (start 100 72.7) (end 101.9 72.7) (width 0.5) (layer "F.Cu") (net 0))
 (segment (start 112.245 70.755) (end 111.125 70.755) (width 0.5) (layer "F.Cu") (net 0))
 (segment (start 113.66 82.86) (end 113.4 82.6) (width 0.5) (layer "F.Cu") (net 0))
 (segment (start 104.3375 72.025) (end 106.824 72.025) (width 0.6) (layer "F.Cu") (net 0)))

